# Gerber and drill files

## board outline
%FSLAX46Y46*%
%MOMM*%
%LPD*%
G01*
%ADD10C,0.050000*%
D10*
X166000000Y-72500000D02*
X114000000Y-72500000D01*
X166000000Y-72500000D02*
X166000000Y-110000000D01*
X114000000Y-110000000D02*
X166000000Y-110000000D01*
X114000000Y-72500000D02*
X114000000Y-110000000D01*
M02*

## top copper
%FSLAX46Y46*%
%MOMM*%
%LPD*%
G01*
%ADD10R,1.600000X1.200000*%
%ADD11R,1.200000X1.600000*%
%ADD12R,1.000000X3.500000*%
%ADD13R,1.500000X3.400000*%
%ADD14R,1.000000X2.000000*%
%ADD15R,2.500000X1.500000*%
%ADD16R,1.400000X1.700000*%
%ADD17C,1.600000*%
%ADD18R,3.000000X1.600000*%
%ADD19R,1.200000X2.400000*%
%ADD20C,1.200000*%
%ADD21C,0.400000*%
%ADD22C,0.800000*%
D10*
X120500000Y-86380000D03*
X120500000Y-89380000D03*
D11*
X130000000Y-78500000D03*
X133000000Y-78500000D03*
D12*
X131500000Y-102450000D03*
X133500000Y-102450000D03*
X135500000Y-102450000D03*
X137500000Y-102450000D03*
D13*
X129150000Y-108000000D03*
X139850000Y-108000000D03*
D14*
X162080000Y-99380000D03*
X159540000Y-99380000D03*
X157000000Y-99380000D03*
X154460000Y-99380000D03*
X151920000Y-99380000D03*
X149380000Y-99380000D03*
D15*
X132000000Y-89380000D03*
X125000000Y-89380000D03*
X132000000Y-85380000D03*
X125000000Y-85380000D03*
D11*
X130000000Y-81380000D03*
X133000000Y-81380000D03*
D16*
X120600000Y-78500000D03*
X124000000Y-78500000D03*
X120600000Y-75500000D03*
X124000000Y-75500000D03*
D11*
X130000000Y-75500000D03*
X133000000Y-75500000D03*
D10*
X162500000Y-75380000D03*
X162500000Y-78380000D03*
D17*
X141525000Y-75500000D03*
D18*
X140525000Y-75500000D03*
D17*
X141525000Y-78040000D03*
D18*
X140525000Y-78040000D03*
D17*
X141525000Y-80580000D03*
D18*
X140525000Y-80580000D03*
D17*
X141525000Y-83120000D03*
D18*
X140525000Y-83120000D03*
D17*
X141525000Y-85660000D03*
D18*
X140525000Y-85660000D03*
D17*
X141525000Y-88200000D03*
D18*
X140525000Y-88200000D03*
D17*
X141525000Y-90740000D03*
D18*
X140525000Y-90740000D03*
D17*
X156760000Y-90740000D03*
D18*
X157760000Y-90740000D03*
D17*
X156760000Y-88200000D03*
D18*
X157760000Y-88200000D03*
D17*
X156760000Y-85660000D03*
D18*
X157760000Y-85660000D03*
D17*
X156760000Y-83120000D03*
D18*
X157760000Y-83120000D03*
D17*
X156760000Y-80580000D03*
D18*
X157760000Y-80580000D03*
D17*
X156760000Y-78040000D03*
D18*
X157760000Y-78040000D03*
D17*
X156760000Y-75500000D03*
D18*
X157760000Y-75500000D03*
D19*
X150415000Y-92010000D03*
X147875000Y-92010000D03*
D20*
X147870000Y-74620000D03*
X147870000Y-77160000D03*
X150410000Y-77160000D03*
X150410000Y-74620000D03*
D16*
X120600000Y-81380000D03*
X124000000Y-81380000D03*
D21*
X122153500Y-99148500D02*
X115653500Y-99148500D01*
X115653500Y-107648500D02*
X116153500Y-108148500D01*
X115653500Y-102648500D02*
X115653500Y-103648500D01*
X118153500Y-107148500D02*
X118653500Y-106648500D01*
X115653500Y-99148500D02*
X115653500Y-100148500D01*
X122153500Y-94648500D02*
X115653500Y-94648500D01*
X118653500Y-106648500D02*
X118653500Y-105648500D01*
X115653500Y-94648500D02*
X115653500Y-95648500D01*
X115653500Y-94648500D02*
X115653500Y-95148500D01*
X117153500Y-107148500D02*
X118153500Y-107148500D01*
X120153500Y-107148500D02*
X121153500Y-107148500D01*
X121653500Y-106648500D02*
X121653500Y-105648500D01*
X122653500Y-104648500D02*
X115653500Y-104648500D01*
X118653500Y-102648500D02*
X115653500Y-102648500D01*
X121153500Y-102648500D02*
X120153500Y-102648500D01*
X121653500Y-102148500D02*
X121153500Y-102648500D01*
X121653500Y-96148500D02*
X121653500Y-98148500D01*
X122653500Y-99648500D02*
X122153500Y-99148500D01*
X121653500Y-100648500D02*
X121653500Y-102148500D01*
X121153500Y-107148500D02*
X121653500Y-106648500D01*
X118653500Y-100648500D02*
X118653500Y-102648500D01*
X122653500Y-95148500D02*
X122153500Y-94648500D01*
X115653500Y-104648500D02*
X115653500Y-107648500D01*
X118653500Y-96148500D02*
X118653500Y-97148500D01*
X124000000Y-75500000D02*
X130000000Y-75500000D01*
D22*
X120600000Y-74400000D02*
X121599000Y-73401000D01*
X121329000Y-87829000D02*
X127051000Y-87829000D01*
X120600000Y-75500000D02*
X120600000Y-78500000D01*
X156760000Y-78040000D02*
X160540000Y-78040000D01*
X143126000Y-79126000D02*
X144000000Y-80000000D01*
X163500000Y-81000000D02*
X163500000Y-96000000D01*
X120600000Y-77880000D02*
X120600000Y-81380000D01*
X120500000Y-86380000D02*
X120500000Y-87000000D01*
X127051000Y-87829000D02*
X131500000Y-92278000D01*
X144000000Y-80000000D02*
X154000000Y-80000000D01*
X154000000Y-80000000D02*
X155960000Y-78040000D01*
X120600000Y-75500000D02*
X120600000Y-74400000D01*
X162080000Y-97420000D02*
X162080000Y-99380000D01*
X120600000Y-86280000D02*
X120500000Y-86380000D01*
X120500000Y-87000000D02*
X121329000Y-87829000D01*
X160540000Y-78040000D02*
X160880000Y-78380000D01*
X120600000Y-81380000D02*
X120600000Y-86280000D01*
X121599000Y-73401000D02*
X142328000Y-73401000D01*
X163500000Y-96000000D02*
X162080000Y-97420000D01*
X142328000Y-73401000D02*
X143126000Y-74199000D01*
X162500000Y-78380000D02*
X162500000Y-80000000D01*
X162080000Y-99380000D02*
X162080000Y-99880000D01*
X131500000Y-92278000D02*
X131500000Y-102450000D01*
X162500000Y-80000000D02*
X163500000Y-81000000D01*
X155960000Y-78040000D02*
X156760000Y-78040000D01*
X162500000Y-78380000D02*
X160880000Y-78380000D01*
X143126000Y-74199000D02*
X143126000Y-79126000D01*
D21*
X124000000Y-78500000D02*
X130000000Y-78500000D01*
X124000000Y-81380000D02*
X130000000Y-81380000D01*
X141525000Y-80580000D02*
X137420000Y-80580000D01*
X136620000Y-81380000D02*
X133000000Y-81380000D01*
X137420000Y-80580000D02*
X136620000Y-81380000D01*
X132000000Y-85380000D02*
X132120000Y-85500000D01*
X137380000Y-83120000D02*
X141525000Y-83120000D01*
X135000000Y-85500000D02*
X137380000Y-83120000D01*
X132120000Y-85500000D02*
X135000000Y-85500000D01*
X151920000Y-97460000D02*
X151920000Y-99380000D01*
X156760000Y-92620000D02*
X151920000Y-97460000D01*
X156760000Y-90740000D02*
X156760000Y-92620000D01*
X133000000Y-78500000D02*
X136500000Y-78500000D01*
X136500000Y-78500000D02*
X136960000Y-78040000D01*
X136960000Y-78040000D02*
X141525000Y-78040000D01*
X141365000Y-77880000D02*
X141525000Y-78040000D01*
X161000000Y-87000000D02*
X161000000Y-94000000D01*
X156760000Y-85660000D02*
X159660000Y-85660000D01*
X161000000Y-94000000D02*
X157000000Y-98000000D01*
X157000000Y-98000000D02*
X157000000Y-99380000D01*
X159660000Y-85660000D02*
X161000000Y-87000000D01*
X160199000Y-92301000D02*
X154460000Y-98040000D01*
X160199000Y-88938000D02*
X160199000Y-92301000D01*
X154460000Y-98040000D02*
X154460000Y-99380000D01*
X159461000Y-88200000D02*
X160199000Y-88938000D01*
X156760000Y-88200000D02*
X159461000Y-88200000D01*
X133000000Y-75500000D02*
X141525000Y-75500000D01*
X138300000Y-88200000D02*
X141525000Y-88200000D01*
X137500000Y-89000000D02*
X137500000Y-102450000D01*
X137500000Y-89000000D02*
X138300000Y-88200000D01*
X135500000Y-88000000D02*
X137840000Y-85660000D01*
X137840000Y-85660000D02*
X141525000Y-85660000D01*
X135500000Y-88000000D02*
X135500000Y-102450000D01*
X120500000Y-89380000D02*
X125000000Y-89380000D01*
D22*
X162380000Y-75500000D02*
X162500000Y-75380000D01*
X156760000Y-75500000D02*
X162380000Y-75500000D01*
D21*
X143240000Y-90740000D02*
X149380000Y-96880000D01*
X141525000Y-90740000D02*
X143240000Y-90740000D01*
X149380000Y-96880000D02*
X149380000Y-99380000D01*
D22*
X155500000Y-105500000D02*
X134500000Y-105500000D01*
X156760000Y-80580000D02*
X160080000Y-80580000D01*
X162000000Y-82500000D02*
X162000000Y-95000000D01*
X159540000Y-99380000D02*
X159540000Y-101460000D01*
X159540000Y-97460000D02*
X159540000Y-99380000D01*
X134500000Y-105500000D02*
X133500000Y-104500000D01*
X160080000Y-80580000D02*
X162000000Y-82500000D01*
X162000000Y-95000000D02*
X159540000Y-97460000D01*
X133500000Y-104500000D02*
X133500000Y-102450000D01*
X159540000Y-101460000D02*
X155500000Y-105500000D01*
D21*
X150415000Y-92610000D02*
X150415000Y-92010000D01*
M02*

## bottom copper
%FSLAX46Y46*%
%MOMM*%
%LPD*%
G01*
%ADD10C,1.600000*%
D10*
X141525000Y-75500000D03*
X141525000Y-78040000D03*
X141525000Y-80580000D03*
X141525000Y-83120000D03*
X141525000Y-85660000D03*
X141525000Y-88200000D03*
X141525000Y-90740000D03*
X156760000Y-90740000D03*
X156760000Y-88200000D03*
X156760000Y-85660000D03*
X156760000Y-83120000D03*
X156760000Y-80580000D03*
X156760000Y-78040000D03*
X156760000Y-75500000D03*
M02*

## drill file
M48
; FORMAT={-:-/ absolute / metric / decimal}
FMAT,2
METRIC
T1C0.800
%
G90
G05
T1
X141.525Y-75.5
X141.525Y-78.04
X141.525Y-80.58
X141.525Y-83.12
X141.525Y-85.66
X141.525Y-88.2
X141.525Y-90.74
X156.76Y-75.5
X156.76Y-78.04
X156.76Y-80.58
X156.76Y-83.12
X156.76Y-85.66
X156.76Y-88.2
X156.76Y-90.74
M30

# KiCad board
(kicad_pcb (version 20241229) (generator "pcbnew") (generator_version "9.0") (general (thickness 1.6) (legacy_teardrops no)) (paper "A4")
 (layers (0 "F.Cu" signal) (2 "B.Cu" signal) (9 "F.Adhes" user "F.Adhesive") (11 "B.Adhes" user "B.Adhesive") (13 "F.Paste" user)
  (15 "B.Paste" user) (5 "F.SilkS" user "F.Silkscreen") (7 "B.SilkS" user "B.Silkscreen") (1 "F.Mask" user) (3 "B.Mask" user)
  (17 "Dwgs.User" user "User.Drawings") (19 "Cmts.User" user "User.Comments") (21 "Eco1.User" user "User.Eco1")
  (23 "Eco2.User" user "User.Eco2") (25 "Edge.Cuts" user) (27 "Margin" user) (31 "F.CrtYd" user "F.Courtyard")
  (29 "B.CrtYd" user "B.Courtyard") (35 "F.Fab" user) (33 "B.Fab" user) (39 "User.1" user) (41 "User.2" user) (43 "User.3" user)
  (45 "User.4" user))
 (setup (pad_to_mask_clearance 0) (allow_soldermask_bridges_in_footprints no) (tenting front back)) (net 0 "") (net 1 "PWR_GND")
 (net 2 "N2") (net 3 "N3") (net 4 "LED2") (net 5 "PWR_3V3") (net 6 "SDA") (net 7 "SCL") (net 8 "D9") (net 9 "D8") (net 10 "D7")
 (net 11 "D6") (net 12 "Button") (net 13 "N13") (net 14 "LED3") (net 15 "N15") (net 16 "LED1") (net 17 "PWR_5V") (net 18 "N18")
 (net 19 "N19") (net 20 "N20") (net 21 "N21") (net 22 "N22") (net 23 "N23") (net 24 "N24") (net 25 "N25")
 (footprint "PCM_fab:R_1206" (layer "F.Cu") (at 120.5 87.88 -90)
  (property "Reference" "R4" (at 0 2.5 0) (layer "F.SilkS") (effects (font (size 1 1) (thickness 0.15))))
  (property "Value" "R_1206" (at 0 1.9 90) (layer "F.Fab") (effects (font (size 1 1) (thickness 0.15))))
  (pad "1" smd rect (at -1.5 0 270) (size 1.2 1.6) (layers "F.Cu" "F.Mask" "F.Paste") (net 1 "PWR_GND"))
  (pad "2" smd rect (at 1.5 0 270) (size 1.2 1.6) (layers "F.Cu" "F.Mask" "F.Paste") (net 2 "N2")))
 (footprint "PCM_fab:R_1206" (layer "F.Cu") (at 131.5 78.5)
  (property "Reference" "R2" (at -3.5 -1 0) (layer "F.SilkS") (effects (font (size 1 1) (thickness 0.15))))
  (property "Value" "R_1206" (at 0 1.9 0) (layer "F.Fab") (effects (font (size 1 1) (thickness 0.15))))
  (pad "1" smd rect (at -1.5 0) (size 1.2 1.6) (layers "F.Cu" "F.Mask" "F.Paste") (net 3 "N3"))
  (pad "2" smd rect (at 1.5 0) (size 1.2 1.6) (layers "F.Cu" "F.Mask" "F.Paste") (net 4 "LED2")))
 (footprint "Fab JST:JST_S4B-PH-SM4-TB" (layer "F.Cu") (at 134.5 105.2)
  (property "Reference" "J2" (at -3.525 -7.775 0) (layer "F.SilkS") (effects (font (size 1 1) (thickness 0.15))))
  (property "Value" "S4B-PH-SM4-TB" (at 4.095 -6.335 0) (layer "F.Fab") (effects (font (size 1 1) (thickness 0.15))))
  (pad "1" smd rect (at -3 -2.75) (size 1 3.5) (layers "F.Cu" "F.Mask" "F.Paste") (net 1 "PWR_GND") (solder_mask_margin 0.102))
  (pad "2" smd rect (at -1 -2.75) (size 1 3.5) (layers "F.Cu" "F.Mask" "F.Paste") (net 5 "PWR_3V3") (solder_mask_margin 0.102))
  (pad "3" smd rect (at 1 -2.75) (size 1 3.5) (layers "F.Cu" "F.Mask" "F.Paste") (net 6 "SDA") (solder_mask_margin 0.102))
  (pad "4" smd rect (at 3 -2.75) (size 1 3.5) (layers "F.Cu" "F.Mask" "F.Paste") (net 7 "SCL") (solder_mask_margin 0.102))
  (pad "SH1" smd rect (at -5.35 2.8) (size 1.5 3.4) (layers "F.Cu" "F.Mask" "F.Paste") (solder_mask_margin 0.102))
  (pad "SH2" smd rect (at 5.35 2.8) (size 1.5 3.4) (layers "F.Cu" "F.Mask" "F.Paste") (solder_mask_margin 0.102)))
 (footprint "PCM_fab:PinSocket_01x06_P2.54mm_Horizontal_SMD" (layer "F.Cu") (at 162.08 99.38 -90)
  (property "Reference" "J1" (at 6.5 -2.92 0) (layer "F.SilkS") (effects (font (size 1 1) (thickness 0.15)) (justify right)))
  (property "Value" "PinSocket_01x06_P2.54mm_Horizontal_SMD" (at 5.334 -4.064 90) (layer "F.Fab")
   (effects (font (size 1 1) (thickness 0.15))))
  (pad "1" smd rect (at 0 0 270) (size 2 1) (layers "F.Cu" "F.Mask" "F.Paste") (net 1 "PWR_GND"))
  (pad "2" smd rect (at 0 2.54 270) (size 2 1) (layers "F.Cu" "F.Mask" "F.Paste") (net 5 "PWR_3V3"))
  (pad "3" smd rect (at 0 5.08 270) (size 2 1) (layers "F.Cu" "F.Mask" "F.Paste") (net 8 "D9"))
  (pad "4" smd rect (at 0 7.62 270) (size 2 1) (layers "F.Cu" "F.Mask" "F.Paste") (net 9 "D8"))
  (pad "5" smd rect (at 0 10.16 270) (size 2 1) (layers "F.Cu" "F.Mask" "F.Paste") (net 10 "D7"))
  (pad "6" smd rect (at 0 12.7 270) (size 2 1) (layers "F.Cu" "F.Mask" "F.Paste") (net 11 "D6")))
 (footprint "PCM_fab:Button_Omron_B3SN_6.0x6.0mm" (layer "F.Cu") (at 128.5 87.38 180)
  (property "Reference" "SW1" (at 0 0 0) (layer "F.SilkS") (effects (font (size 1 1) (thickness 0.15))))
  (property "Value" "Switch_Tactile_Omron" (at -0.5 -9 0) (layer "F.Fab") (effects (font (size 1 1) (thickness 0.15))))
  (pad "1" smd rect (at -3.5 -2 180) (size 2.5 1.5) (layers "F.Cu" "F.Mask" "F.Paste") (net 2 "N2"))
  (pad "1" smd rect (at 3.5 -2 180) (size 2.5 1.5) (layers "F.Cu" "F.Mask" "F.Paste") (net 2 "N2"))
  (pad "2" smd rect (at -3.5 2 180) (size 2.5 1.5) (layers "F.Cu" "F.Mask" "F.Paste") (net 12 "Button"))
  (pad "2" smd rect (at 3.5 2 180) (size 2.5 1.5) (layers "F.Cu" "F.Mask" "F.Paste") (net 12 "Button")))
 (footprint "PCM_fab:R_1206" (layer "F.Cu") (at 131.5 81.38)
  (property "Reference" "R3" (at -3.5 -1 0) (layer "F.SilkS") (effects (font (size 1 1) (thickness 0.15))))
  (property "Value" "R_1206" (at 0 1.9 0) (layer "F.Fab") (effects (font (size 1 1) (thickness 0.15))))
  (pad "1" smd rect (at -1.5 0) (size 1.2 1.6) (layers "F.Cu" "F.Mask" "F.Paste") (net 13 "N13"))
  (pad "2" smd rect (at 1.5 0) (size 1.2 1.6) (layers "F.Cu" "F.Mask" "F.Paste") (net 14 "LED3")))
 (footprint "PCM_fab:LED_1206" (layer "F.Cu") (at 122.3 78.5)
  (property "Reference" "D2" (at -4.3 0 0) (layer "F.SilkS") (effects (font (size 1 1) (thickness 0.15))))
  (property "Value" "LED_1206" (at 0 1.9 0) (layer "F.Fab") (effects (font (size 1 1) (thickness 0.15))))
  (pad "1" smd rect (at -1.7 0) (size 1.4 1.7) (layers "F.Cu" "F.Mask" "F.Paste") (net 1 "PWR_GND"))
  (pad "2" smd rect (at 1.7 0) (size 1.4 1.7) (layers "F.Cu" "F.Mask" "F.Paste") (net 3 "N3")))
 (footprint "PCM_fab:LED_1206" (layer "F.Cu") (at 122.3 75.5)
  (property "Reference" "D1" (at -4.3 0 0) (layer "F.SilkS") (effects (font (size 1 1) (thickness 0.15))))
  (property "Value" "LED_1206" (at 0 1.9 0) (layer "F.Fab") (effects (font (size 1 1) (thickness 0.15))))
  (pad "1" smd rect (at -1.7 0) (size 1.4 1.7) (layers "F.Cu" "F.Mask" "F.Paste") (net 1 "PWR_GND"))
  (pad "2" smd rect (at 1.7 0) (size 1.4 1.7) (layers "F.Cu" "F.Mask" "F.Paste") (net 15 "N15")))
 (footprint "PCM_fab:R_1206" (layer "F.Cu") (at 131.5 75.5)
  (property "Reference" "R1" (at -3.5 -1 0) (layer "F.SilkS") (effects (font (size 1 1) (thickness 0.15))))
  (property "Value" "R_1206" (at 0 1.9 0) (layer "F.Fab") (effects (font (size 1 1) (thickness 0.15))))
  (pad "1" smd rect (at -1.5 0) (size 1.2 1.6) (layers "F.Cu" "F.Mask" "F.Paste") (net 15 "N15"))
  (pad "2" smd rect (at 1.5 0) (size 1.2 1.6) (layers "F.Cu" "F.Mask" "F.Paste") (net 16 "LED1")))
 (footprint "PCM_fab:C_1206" (layer "F.Cu") (at 162.5 76.88 -90)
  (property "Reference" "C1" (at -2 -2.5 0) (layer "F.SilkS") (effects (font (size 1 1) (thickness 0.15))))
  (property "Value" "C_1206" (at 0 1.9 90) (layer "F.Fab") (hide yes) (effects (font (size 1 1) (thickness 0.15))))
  (pad "1" smd rect (at -1.5 0 270) (size 1.2 1.6) (layers "F.Cu" "F.Mask" "F.Paste") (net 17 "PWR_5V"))
  (pad "2" smd rect (at 1.5 0 270) (size 1.2 1.6) (layers "F.Cu" "F.Mask" "F.Paste") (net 1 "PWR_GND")))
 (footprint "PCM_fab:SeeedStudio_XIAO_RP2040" (layer "F.Cu") (at 149.14 83.12)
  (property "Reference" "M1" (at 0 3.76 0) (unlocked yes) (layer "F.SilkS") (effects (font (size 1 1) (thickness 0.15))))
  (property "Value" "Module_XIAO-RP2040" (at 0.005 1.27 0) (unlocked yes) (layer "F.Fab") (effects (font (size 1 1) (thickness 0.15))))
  (pad "1" thru_hole circle (at -7.615 -7.62) (size 1.6 1.6) (drill 0.8) (layers "*.Cu" "*.Mask") (remove_unused_layers no) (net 16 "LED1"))
  (pad "1" smd rect (at -7.615 -7.62) (size 3 1.6) (drill (offset -1 0)) (layers "F.Cu" "F.Mask" "F.Paste") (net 16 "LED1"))
  (pad "2" thru_hole circle (at -7.615 -5.08) (size 1.6 1.6) (drill 0.8) (layers "*.Cu" "*.Mask") (remove_unused_layers no) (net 4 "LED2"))
  (pad "2" smd rect (at -7.615 -5.08) (size 3 1.6) (drill (offset -1 0)) (layers "F.Cu" "F.Mask" "F.Paste") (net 4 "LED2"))
  (pad "3" thru_hole circle (at -7.615 -2.54) (size 1.6 1.6) (drill 0.8) (layers "*.Cu" "*.Mask") (remove_unused_layers no) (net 14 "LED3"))
  (pad "3" smd rect (at -7.615 -2.54) (size 3 1.6) (drill (offset -1 0)) (layers "F.Cu" "F.Mask" "F.Paste") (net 14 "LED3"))
  (pad "4" thru_hole circle (at -7.615 0) (size 1.6 1.6) (drill 0.8) (layers "*.Cu" "*.Mask") (remove_unused_layers no) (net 12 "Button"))
  (pad "4" smd rect (at -7.615 0) (size 3 1.6) (drill (offset -1 0)) (layers "F.Cu" "F.Mask" "F.Paste") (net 12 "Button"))
  (pad "5" thru_hole circle (at -7.615 2.54) (size 1.6 1.6) (drill 0.8) (layers "*.Cu" "*.Mask") (remove_unused_layers no) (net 6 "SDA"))
  (pad "5" smd rect (at -7.615 2.54) (size 3 1.6) (drill (offset -1 0)) (layers "F.Cu" "F.Mask" "F.Paste") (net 6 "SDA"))
  (pad "6" thru_hole circle (at -7.615 5.08) (size 1.6 1.6) (drill 0.8) (layers "*.Cu" "*.Mask") (remove_unused_layers no) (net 7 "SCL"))
  (pad "6" smd rect (at -7.615 5.08) (size 3 1.6) (drill (offset -1 0)) (layers "F.Cu" "F.Mask" "F.Paste") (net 7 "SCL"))
  (pad "7" thru_hole circle (at -7.615 7.62) (size 1.6 1.6) (drill 0.8) (layers "*.Cu" "*.Mask") (remove_unused_layers no) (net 11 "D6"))
  (pad "7" smd rect (at -7.615 7.62) (size 3 1.6) (drill (offset -1 0)) (layers "F.Cu" "F.Mask" "F.Paste") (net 11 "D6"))
  (pad "8" thru_hole circle (at 7.62 7.62) (size 1.6 1.6) (drill 0.8) (layers "*.Cu" "*.Mask") (remove_unused_layers no) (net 10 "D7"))
  (pad "8" smd rect (at 7.62 7.62) (size 3 1.6) (drill (offset 1 0)) (layers "F.Cu" "F.Mask" "F.Paste") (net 10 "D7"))
  (pad "9" thru_hole circle (at 7.62 5.08) (size 1.6 1.6) (drill 0.8) (layers "*.Cu" "*.Mask") (remove_unused_layers no) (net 9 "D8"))
  (pad "9" smd rect (at 7.62 5.08) (size 3 1.6) (drill (offset 1 0)) (layers "F.Cu" "F.Mask" "F.Paste") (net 9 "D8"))
  (pad "10" thru_hole circle (at 7.62 2.54) (size 1.6 1.6) (drill 0.8) (layers "*.Cu" "*.Mask") (remove_unused_layers no) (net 8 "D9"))
  (pad "10" smd rect (at 7.62 2.54) (size 3 1.6) (drill (offset 1 0)) (layers "F.Cu" "F.Mask" "F.Paste") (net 8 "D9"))
  (pad "11" thru_hole circle (at 7.62 0) (size 1.6 1.6) (drill 0.8) (layers "*.Cu" "*.Mask") (remove_unused_layers no) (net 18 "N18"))
  (pad "11" smd rect (at 7.62 0) (size 3 1.6) (drill (offset 1 0)) (layers "F.Cu" "F.Mask" "F.Paste") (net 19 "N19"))
  (pad "12" thru_hole circle (at 7.62 -2.54) (size 1.6 1.6) (drill 0.8) (layers "*.Cu" "*.Mask") (remove_unused_layers no) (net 5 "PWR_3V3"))
  (pad "12" smd rect (at 7.62 -2.54) (size 3 1.6) (drill (offset 1 0)) (layers "F.Cu" "F.Mask" "F.Paste") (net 5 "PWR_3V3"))
  (pad "13" thru_hole circle (at 7.62 -5.08) (size 1.6 1.6) (drill 0.8) (layers "*.Cu" "*.Mask") (remove_unused_layers no) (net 1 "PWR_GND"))
  (pad "13" smd rect (at 7.62 -5.08) (size 3 1.6) (drill (offset 1 0)) (layers "F.Cu" "F.Mask" "F.Paste") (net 1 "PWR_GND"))
  (pad "14" thru_hole circle (at 7.62 -7.62) (size 1.6 1.6) (drill 0.8) (layers "*.Cu" "*.Mask") (remove_unused_layers no) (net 17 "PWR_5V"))
  (pad "14" smd rect (at 7.62 -7.62) (size 3 1.6) (drill (offset 1 0)) (layers "F.Cu" "F.Mask" "F.Paste") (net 17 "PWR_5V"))
  (pad "15" smd rect (at 1.275 8.89 270) (size 2.4 1.2) (layers "F.Cu" "F.Mask" "F.Paste") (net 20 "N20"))
  (pad "16" smd rect (at -1.265 8.89 270) (size 2.4 1.2) (layers "F.Cu" "F.Mask" "F.Paste") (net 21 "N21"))
  (pad "17" smd circle (at -1.27 -8.5) (size 1.2 1.2) (layers "F.Cu" "F.Mask" "F.Paste") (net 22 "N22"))
  (pad "18" smd circle (at -1.27 -5.96) (size 1.2 1.2) (layers "F.Cu" "F.Mask" "F.Paste") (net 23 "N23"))
  (pad "19" smd circle (at 1.27 -5.96) (size 1.2 1.2) (layers "F.Cu" "F.Mask" "F.Paste") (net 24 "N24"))
  (pad "20" smd circle (at 1.27 -8.5) (size 1.2 1.2) (layers "F.Cu" "F.Mask" "F.Paste") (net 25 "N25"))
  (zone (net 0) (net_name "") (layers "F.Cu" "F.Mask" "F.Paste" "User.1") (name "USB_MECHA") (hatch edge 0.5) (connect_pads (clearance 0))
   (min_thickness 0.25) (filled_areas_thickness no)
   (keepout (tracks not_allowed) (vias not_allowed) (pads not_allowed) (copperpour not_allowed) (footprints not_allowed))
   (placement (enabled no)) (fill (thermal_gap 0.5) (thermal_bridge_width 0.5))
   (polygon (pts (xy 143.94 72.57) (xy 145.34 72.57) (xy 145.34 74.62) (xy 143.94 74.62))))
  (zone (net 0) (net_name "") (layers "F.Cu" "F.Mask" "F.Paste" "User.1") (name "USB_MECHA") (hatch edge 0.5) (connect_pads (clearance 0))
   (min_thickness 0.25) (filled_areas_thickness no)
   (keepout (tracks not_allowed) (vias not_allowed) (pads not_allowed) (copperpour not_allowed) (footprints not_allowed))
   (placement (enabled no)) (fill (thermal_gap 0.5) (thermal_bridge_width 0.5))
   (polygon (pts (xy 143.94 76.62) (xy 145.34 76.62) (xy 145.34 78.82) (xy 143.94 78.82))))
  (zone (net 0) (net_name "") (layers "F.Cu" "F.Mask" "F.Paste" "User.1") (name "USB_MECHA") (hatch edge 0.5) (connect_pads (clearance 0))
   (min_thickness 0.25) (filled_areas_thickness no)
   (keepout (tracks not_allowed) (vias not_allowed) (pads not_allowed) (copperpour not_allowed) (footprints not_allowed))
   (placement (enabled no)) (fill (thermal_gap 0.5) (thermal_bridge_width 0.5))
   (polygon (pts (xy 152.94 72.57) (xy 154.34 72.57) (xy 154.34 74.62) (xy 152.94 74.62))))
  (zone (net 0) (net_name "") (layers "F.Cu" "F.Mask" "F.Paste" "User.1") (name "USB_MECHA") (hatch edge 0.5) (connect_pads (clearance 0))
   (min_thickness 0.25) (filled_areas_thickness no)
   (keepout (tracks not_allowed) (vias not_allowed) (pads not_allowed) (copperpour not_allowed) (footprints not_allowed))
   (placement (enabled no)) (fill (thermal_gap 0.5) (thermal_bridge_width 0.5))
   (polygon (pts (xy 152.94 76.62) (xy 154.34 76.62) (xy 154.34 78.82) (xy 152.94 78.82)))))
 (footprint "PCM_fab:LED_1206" (layer "F.Cu") (at 122.3 81.38)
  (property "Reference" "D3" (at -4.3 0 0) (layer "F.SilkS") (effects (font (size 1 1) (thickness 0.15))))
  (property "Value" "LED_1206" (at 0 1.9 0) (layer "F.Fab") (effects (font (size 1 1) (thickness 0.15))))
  (pad "1" smd rect (at -1.7 0) (size 1.4 1.7) (layers "F.Cu" "F.Mask" "F.Paste") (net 1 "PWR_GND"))
  (pad "2" smd rect (at 1.7 0) (size 1.4 1.7) (layers "F.Cu" "F.Mask" "F.Paste") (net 13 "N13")))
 (gr_line (start 166 72.5) (end 114 72.5) (stroke (width 0.05) (type default)) (layer "Edge.Cuts"))
 (gr_line (start 166 72.5) (end 166 110) (stroke (width 0.05) (type default)) (layer "Edge.Cuts"))
 (gr_line (start 114 110) (end 166 110) (stroke (width 0.05) (type default)) (layer "Edge.Cuts"))
 (gr_line (start 114 72.5) (end 114 110) (stroke (width 0.05) (type default)) (layer "Edge.Cuts"))
 (segment (start 122.1535 99.1485) (end 115.6535 99.1485) (width 0.4) (layer "F.Cu") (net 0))
 (segment (start 115.6535 107.6485) (end 116.1535 108.1485) (width 0.4) (layer "F.Cu") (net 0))
 (segment (start 115.6535 102.6485) (end 115.6535 103.6485) (width 0.4) (layer "F.Cu") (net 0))
 (segment (start 118.1535 107.1485) (end 118.6535 106.6485) (width 0.4) (layer "F.Cu") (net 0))
 (segment (start 115.6535 99.1485) (end 115.6535 100.1485) (width 0.4) (layer "F.Cu") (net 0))
 (segment (start 122.1535 94.6485) (end 115.6535 94.6485) (width 0.4) (layer "F.Cu") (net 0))
 (segment (start 118.6535 106.6485) (end 118.6535 105.6485) (width 0.4) (layer "F.Cu") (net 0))
 (segment (start 115.6535 94.6485) (end 115.6535 95.6485) (width 0.4) (layer "F.Cu") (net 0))
 (segment (start 115.6535 94.6485) (end 115.6535 95.1485) (width 0.4) (layer "F.Cu") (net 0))
 (segment (start 117.1535 107.1485) (end 118.1535 107.1485) (width 0.4) (layer "F.Cu") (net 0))
 (segment (start 120.1535 107.1485) (end 121.1535 107.1485) (width 0.4) (layer "F.Cu") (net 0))
 (segment (start 121.6535 106.6485) (end 121.6535 105.6485) (width 0.4) (layer "F.Cu") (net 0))
 (segment (start 122.6535 104.6485) (end 115.6535 104.6485) (width 0.4) (layer "F.Cu") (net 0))
 (segment (start 118.6535 102.6485) (end 115.6535 102.6485) (width 0.4) (layer "F.Cu") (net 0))
 (segment (start 121.1535 102.6485) (end 120.1535 102.6485) (width 0.4) (layer "F.Cu") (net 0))
 (segment (start 121.6535 102.1485) (end 121.1535 102.6485) (width 0.4) (layer "F.Cu") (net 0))
 (segment (start 121.6535 96.1485) (end 121.6535 98.1485) (width 0.4) (layer "F.Cu") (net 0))
 (segment (start 122.6535 99.6485) (end 122.1535 99.1485) (width 0.4) (layer "F.Cu") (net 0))
 (segment (start 121.6535 100.6485) (end 121.6535 102.1485) (width 0.4) (layer "F.Cu") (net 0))
 (segment (start 121.1535 107.1485) (end 121.6535 106.6485) (width 0.4) (layer "F.Cu") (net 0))
 (segment (start 118.6535 100.6485) (end 118.6535 102.6485) (width 0.4) (layer "F.Cu") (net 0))
 (segment (start 122.6535 95.1485) (end 122.1535 94.6485) (width 0.4) (layer "F.Cu") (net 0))
 (segment (start 115.6535 104.6485) (end 115.6535 107.6485) (width 0.4) (layer "F.Cu") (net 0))
 (segment (start 118.6535 96.1485) (end 118.6535 97.1485) (width 0.4) (layer "F.Cu") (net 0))
 (segment (start 124 75.5) (end 130 75.5) (width 0.4) (layer "F.Cu") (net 15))
 (segment (start 120.6 74.4) (end 121.599 73.401) (width 0.8) (layer "F.Cu") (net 1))
 (segment (start 121.329 87.829) (end 127.051 87.829) (width 0.8) (layer "F.Cu") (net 1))
 (segment (start 120.6 75.5) (end 120.6 78.5) (width 0.8) (layer "F.Cu") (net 1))
 (segment (start 156.76 78.04) (end 160.54 78.04) (width 0.8) (layer "F.Cu") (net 1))
 (segment (start 143.126 79.126) (end 144 80) (width 0.8) (layer "F.Cu") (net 1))
 (segment (start 163.5 81) (end 163.5 96) (width 0.8) (layer "F.Cu") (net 1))
 (segment (start 120.6 77.88) (end 120.6 81.38) (width 0.8) (layer "F.Cu") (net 1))
 (segment (start 120.5 86.38) (end 120.5 87) (width 0.8) (layer "F.Cu") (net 1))
 (segment (start 127.051 87.829) (end 131.5 92.278) (width 0.8) (layer "F.Cu") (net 1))
 (segment (start 144 80) (end 154 80) (width 0.8) (layer "F.Cu") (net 1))
 (segment (start 154 80) (end 155.96 78.04) (width 0.8) (layer "F.Cu") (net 1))
 (segment (start 120.6 75.5) (end 120.6 74.4) (width 0.8) (layer "F.Cu") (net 1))
 (segment (start 162.08 97.42) (end 162.08 99.38) (width 0.8) (layer "F.Cu") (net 1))
 (segment (start 120.6 86.28) (end 120.5 86.38) (width 0.8) (layer "F.Cu") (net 1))
 (segment (start 120.5 87) (end 121.329 87.829) (width 0.8) (layer "F.Cu") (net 1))
 (segment (start 160.54 78.04) (end 160.88 78.38) (width 0.8) (layer "F.Cu") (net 1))
 (segment (start 120.6 81.38) (end 120.6 86.28) (width 0.8) (layer "F.Cu") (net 1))
 (segment (start 121.599 73.401) (end 142.328 73.401) (width 0.8) (layer "F.Cu") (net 1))
 (segment (start 163.5 96) (end 162.08 97.42) (width 0.8) (layer "F.Cu") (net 1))
 (segment (start 142.328 73.401) (end 143.126 74.199) (width 0.8) (layer "F.Cu") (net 1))
 (segment (start 162.5 78.38) (end 162.5 80) (width 0.8) (layer "F.Cu") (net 1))
 (segment (start 162.08 99.38) (end 162.08 99.88) (width 0.8) (layer "F.Cu") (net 1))
 (segment (start 131.5 92.278) (end 131.5 102.45) (width 0.8) (layer "F.Cu") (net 1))
 (segment (start 162.5 80) (end 163.5 81) (width 0.8) (layer "F.Cu") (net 1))
 (segment (start 155.96 78.04) (end 156.76 78.04) (width 0.8) (layer "F.Cu") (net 1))
 (segment (start 162.5 78.38) (end 160.88 78.38) (width 0.8) (layer "F.Cu") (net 1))
 (segment (start 143.126 74.199) (end 143.126 79.126) (width 0.8) (layer "F.Cu") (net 1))
 (segment (start 124 78.5) (end 130 78.5) (width 0.4) (layer "F.Cu") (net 3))
 (segment (start 124 81.38) (end 130 81.38) (width 0.4) (layer "F.Cu") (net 13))
 (segment (start 141.525 80.58) (end 137.42 80.58) (width 0.4) (layer "F.Cu") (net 14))
 (segment (start 136.62 81.38) (end 133 81.38) (width 0.4) (layer "F.Cu") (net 14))
 (segment (start 137.42 80.58) (end 136.62 81.38) (width 0.4) (layer "F.Cu") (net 14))
 (segment (start 132 85.38) (end 132.12 85.5) (width 0.4) (layer "F.Cu") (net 12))
 (segment (start 137.38 83.12) (end 141.525 83.12) (width 0.4) (layer "F.Cu") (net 12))
 (segment (start 135 85.5) (end 137.38 83.12) (width 0.4) (layer "F.Cu") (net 12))
 (segment (start 132.12 85.5) (end 135 85.5) (width 0.4) (layer "F.Cu") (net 12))
 (segment (start 151.92 97.46) (end 151.92 99.38) (width 0.4) (layer "F.Cu") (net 10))
 (segment (start 156.76 92.62) (end 151.92 97.46) (width 0.4) (layer "F.Cu") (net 10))
 (segment (start 156.76 90.74) (end 156.76 92.62) (width 0.4) (layer "F.Cu") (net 10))
 (segment (start 133 78.5) (end 136.5 78.5) (width 0.4) (layer "F.Cu") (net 4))
 (segment (start 136.5 78.5) (end 136.96 78.04) (width 0.4) (layer "F.Cu") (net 4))
 (segment (start 136.96 78.04) (end 141.525 78.04) (width 0.4) (layer "F.Cu") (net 4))
 (segment (start 141.365 77.88) (end 141.525 78.04) (width 0.4) (layer "F.Cu") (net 4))
 (segment (start 161 87) (end 161 94) (width 0.4) (layer "F.Cu") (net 8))
 (segment (start 156.76 85.66) (end 159.66 85.66) (width 0.4) (layer "F.Cu") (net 8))
 (segment (start 161 94) (end 157 98) (width 0.4) (layer "F.Cu") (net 8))
 (segment (start 157 98) (end 157 99.38) (width 0.4) (layer "F.Cu") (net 8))
 (segment (start 159.66 85.66) (end 161 87) (width 0.4) (layer "F.Cu") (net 8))
 (segment (start 160.199 92.301) (end 154.46 98.04) (width 0.4) (layer "F.Cu") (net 9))
 (segment (start 160.199 88.938) (end 160.199 92.301) (width 0.4) (layer "F.Cu") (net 9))
 (segment (start 154.46 98.04) (end 154.46 99.38) (width 0.4) (layer "F.Cu") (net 9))
 (segment (start 159.461 88.2) (end 160.199 88.938) (width 0.4) (layer "F.Cu") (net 9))
 (segment (start 156.76 88.2) (end 159.461 88.2) (width 0.4) (layer "F.Cu") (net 9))
 (segment (start 133 75.5) (end 141.525 75.5) (width 0.4) (layer "F.Cu") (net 16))
 (segment (start 138.3 88.2) (end 141.525 88.2) (width 0.4) (layer "F.Cu") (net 7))
 (segment (start 137.5 89) (end 137.5 102.45) (width 0.4) (layer "F.Cu") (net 7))
 (segment (start 137.5 89) (end 138.3 88.2) (width 0.4) (layer "F.Cu") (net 7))
 (segment (start 135.5 88) (end 137.84 85.66) (width 0.4) (layer "F.Cu") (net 6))
 (segment (start 137.84 85.66) (end 141.525 85.66) (width 0.4) (layer "F.Cu") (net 6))
 (segment (start 135.5 88) (end 135.5 102.45) (width 0.4) (layer "F.Cu") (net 6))
 (segment (start 120.5 89.38) (end 125 89.38) (width 0.4) (layer "F.Cu") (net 2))
 (segment (start 162.38 75.5) (end 162.5 75.38) (width 0.8) (layer "F.Cu") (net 17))
 (segment (start 156.76 75.5) (end 162.38 75.5) (width 0.8) (layer "F.Cu") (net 17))
 (segment (start 143.24 90.74) (end 149.38 96.88) (width 0.4) (layer "F.Cu") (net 11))
 (segment (start 141.525 90.74) (end 143.24 90.74) (width 0.4) (layer "F.Cu") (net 11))
 (segment (start 149.38 96.88) (end 149.38 99.38) (width 0.4) (layer "F.Cu") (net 11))
 (segment (start 155.5 105.5) (end 134.5 105.5) (width 0.8) (layer "F.Cu") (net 5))
 (segment (start 156.76 80.58) (end 160.08 80.58) (width 0.8) (layer "F.Cu") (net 5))
 (segment (start 162 82.5) (end 162 95) (width 0.8) (layer "F.Cu") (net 5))
 (segment (start 159.54 99.38) (end 159.54 101.46) (width 0.8) (layer "F.Cu") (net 5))
 (segment (start 159.54 97.46) (end 159.54 99.38) (width 0.8) (layer "F.Cu") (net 5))
 (segment (start 134.5 105.5) (end 133.5 104.5) (width 0.8) (layer "F.Cu") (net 5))
 (segment (start 160.08 80.58) (end 162 82.5) (width 0.8) (layer "F.Cu") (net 5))
 (segment (start 162 95) (end 159.54 97.46) (width 0.8) (layer "F.Cu") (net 5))
 (segment (start 133.5 104.5) (end 133.5 102.45) (width 0.8) (layer "F.Cu") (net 5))
 (segment (start 159.54 101.46) (end 155.5 105.5) (width 0.8) (layer "F.Cu") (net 5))
 (segment (start 150.415 92.61) (end 150.415 92.01) (width 0.4) (layer "F.Cu") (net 20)))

